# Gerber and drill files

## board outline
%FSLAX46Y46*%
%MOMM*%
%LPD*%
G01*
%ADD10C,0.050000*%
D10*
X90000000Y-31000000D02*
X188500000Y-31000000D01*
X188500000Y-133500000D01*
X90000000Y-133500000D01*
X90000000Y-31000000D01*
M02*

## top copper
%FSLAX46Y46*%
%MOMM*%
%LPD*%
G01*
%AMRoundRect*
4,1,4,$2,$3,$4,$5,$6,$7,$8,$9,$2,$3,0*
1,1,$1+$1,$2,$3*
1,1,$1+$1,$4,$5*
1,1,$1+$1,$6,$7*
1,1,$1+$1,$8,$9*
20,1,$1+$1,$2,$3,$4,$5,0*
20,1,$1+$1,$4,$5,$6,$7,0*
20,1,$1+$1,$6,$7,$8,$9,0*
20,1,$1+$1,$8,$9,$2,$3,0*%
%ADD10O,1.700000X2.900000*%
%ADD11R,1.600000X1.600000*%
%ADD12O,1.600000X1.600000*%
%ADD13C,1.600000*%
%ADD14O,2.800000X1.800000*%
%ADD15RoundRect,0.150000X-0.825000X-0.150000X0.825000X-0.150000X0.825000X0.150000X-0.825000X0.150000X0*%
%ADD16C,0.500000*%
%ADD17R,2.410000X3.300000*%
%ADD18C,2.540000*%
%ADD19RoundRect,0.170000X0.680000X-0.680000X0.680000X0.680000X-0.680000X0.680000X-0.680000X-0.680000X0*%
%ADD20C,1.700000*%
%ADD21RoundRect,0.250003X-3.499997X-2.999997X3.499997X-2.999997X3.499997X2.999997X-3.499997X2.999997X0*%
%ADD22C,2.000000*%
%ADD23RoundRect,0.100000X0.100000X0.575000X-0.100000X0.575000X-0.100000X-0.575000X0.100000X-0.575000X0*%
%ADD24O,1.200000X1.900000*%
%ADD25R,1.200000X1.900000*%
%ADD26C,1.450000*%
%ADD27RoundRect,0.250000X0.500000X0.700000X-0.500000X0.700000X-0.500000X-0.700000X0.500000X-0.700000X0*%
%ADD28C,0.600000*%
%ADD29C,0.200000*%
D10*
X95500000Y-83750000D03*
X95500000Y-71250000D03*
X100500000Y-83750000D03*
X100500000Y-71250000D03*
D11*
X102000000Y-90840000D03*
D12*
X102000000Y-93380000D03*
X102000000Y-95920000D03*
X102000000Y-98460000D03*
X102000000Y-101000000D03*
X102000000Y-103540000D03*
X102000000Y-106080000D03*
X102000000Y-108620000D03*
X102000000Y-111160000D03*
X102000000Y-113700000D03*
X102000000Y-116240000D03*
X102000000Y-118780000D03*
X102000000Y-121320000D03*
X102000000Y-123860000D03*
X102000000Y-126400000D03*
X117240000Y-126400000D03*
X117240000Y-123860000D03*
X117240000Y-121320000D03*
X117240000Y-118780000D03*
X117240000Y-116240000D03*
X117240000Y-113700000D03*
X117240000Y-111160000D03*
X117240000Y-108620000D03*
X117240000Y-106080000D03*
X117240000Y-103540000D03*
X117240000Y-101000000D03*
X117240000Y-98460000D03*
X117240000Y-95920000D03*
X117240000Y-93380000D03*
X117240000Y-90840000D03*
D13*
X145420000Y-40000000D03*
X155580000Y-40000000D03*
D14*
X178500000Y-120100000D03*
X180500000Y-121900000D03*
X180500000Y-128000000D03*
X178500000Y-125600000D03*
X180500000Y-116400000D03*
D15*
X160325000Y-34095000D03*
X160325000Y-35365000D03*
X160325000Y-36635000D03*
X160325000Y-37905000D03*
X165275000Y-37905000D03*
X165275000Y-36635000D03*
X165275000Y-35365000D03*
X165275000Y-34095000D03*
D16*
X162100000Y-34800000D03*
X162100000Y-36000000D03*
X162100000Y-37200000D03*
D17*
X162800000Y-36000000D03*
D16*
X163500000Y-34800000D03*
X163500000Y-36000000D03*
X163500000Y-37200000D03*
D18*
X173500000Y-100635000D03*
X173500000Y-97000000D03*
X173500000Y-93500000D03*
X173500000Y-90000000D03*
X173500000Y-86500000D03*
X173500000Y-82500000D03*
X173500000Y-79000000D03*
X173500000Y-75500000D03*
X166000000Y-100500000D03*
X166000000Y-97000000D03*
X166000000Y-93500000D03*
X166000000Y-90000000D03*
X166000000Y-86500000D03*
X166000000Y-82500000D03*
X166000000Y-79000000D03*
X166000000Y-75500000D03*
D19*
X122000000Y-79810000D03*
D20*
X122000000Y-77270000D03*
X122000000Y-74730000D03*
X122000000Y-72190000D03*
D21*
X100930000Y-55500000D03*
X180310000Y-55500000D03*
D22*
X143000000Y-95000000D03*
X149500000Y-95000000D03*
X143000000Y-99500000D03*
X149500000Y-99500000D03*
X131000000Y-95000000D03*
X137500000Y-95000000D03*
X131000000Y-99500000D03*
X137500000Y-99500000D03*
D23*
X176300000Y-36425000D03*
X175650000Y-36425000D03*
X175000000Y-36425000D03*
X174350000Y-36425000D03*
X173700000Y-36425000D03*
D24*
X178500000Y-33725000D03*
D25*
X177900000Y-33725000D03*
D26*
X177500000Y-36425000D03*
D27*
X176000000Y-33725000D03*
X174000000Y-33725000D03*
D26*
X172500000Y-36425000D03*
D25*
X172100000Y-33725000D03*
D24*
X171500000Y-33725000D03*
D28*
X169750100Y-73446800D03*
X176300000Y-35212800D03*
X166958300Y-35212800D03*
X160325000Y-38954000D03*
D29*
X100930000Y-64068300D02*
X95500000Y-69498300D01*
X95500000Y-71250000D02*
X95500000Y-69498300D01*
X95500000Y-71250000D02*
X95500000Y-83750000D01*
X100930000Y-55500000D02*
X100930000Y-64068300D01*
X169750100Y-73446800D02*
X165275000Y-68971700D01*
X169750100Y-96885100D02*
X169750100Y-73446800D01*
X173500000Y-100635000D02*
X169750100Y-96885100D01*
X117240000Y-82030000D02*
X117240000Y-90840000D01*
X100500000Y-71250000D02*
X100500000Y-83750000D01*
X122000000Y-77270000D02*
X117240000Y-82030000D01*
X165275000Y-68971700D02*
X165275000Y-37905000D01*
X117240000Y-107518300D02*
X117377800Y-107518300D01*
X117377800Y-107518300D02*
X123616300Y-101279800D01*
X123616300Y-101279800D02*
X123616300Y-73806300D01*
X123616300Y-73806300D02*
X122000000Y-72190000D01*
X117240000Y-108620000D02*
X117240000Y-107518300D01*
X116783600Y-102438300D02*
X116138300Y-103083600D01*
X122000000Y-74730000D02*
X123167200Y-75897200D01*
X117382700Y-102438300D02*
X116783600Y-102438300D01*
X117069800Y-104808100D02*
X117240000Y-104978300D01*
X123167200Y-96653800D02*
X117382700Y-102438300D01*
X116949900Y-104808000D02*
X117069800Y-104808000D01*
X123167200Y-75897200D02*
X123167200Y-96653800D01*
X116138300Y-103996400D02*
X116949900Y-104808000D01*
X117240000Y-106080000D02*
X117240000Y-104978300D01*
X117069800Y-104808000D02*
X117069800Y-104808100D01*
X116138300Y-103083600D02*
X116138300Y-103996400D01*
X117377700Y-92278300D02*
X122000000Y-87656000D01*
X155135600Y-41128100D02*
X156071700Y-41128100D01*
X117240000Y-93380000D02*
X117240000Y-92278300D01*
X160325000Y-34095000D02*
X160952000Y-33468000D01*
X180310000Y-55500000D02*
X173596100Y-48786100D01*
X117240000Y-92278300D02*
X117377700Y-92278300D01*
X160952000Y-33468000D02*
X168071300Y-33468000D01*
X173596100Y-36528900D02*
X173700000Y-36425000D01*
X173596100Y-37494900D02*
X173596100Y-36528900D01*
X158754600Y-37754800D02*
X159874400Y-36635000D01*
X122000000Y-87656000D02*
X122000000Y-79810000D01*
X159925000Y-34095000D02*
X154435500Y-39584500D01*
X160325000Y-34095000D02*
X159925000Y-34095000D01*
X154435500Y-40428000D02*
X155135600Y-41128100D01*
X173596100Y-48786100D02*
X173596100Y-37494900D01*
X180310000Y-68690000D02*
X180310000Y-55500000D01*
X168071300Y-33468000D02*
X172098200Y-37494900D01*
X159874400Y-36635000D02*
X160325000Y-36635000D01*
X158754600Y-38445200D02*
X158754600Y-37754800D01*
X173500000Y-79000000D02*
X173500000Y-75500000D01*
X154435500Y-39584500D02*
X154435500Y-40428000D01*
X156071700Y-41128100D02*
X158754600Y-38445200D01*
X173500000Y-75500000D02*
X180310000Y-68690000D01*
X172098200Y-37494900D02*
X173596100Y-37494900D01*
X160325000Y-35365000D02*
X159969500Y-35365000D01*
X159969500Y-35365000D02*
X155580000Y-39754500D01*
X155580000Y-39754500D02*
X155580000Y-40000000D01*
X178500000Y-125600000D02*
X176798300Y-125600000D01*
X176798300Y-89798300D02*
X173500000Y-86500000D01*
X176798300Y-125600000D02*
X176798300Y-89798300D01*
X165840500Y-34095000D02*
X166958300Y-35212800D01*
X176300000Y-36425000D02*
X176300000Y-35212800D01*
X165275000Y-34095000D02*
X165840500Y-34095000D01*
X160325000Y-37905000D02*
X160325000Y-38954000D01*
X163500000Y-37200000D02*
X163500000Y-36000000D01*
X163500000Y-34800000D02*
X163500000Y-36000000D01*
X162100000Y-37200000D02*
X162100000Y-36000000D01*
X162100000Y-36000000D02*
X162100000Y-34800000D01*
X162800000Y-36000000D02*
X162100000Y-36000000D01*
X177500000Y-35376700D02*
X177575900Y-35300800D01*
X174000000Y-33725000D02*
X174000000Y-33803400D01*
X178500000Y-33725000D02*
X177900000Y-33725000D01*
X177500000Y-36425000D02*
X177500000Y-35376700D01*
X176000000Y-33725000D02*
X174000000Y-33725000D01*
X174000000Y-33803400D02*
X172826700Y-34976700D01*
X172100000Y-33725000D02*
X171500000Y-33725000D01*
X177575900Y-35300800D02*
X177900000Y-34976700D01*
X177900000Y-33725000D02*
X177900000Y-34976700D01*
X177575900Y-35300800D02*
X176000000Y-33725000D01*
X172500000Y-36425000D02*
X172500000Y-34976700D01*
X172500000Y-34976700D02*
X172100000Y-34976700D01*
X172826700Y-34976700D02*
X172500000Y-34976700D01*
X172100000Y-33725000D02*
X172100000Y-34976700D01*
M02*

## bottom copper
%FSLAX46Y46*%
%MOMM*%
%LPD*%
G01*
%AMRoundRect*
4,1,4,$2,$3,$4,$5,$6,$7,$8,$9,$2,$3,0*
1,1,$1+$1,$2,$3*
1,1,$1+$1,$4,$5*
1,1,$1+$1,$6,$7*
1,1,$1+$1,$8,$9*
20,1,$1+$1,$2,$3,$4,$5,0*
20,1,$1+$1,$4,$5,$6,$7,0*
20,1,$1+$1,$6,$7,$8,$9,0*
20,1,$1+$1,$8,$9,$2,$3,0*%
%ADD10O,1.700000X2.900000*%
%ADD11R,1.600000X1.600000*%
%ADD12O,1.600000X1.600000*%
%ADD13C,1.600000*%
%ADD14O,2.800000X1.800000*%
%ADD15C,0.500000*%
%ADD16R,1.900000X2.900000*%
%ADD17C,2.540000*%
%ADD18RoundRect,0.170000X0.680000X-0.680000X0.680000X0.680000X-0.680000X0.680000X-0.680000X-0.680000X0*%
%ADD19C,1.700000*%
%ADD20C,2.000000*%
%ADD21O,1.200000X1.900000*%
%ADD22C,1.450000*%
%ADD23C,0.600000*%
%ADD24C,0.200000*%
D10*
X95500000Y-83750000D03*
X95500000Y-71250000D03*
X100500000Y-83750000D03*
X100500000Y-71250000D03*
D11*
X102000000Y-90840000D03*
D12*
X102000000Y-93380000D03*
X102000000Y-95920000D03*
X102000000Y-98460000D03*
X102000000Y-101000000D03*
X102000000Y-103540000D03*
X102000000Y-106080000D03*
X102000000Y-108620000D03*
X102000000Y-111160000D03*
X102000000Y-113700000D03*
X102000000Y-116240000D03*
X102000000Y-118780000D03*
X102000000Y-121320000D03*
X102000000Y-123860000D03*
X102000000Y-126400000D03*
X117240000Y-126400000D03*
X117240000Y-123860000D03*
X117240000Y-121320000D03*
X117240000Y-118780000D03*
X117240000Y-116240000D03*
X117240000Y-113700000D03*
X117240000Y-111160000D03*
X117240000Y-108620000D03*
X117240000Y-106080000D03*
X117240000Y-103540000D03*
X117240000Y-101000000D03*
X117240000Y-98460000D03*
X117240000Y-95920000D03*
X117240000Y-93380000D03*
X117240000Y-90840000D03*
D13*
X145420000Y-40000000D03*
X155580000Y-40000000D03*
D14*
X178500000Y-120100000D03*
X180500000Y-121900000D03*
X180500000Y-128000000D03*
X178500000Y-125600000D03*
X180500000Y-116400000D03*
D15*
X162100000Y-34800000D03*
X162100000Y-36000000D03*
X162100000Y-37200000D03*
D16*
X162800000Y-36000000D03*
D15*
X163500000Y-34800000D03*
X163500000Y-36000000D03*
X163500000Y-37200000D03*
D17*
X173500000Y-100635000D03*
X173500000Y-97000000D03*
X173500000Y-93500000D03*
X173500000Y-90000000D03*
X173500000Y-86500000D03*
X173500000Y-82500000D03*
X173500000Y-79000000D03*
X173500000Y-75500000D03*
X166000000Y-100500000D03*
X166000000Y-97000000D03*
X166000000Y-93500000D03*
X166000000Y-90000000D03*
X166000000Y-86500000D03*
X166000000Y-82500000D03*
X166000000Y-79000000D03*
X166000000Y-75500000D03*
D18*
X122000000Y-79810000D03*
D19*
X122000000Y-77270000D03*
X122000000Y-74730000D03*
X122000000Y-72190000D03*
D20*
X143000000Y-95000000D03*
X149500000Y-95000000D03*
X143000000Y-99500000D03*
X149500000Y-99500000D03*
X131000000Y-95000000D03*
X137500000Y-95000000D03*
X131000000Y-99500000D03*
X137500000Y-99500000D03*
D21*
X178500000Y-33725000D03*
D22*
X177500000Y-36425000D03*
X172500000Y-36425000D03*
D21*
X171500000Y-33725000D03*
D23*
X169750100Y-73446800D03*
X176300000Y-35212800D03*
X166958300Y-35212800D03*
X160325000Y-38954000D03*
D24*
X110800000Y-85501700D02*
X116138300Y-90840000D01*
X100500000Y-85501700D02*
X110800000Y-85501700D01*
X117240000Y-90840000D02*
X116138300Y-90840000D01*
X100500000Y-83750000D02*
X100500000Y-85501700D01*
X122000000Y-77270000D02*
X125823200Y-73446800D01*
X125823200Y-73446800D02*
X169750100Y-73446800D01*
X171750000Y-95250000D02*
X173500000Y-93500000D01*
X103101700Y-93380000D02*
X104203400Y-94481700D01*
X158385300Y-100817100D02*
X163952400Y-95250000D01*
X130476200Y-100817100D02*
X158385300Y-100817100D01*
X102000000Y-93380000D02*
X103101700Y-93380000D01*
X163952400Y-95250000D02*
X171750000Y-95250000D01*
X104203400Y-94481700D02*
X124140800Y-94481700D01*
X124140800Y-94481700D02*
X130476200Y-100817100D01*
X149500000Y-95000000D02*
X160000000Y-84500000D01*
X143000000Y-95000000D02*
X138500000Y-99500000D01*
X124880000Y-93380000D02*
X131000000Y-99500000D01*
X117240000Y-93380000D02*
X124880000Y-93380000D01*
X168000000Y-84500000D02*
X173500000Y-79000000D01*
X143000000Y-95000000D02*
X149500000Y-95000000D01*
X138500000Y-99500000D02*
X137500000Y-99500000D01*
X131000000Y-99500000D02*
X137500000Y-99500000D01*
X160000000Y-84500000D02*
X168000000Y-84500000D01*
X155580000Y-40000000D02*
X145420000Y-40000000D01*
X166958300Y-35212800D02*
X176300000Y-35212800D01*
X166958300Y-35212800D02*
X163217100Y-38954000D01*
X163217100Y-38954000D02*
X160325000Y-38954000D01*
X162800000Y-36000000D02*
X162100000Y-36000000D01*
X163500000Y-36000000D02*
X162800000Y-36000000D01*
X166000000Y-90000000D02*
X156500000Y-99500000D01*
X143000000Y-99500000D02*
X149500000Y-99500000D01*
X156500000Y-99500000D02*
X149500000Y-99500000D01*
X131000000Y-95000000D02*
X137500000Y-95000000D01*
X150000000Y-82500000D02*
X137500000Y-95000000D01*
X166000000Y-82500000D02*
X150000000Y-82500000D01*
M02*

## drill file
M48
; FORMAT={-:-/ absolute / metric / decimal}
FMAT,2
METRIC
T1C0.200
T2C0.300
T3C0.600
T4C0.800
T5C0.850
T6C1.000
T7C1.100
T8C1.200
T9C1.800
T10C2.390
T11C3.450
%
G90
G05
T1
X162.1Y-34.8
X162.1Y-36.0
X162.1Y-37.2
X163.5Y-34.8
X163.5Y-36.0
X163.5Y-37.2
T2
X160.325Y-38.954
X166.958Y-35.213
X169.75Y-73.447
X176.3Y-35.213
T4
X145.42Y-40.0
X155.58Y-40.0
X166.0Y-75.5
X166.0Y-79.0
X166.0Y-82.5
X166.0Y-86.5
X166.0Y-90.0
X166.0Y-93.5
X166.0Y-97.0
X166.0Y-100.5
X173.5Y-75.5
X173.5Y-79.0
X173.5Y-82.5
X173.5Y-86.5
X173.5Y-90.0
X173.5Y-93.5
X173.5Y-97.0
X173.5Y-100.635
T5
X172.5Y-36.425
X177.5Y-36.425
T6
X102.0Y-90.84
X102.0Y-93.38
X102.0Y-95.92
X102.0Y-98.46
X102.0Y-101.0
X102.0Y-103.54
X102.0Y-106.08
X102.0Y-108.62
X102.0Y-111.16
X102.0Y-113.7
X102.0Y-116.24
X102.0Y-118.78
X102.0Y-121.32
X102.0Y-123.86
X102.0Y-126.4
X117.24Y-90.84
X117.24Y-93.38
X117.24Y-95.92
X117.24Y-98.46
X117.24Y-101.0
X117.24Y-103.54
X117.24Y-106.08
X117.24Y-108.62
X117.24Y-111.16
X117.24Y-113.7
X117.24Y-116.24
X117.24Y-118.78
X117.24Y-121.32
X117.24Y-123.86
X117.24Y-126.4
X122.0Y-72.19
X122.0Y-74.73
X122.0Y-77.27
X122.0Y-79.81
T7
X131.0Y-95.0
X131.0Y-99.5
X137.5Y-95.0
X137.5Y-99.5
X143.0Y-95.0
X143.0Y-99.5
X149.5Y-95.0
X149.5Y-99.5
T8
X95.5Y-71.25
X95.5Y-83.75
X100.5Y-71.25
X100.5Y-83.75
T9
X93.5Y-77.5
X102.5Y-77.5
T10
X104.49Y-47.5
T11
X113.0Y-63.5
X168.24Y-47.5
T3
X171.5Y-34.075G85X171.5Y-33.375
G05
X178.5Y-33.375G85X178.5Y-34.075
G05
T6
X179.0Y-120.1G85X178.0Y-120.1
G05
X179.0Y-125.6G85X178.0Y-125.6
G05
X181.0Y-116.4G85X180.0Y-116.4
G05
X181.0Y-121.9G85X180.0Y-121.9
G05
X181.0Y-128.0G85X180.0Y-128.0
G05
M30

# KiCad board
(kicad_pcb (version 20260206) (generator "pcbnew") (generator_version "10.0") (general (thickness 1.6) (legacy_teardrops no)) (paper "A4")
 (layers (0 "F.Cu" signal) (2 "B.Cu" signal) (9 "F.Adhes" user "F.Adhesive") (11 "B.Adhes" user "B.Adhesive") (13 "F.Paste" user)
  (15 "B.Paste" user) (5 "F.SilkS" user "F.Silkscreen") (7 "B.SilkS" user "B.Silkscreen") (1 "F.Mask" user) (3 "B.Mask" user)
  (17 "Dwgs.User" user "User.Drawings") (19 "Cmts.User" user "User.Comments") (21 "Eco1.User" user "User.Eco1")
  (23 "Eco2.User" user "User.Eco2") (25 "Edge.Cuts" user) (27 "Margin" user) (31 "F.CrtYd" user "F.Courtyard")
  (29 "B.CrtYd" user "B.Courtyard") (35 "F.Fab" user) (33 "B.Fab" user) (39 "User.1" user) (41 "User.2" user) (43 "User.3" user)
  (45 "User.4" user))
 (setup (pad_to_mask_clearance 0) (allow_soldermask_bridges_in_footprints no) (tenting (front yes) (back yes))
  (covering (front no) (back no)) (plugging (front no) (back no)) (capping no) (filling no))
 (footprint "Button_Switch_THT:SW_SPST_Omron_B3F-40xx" (layer "F.Cu") (at 95.5 83.75 90)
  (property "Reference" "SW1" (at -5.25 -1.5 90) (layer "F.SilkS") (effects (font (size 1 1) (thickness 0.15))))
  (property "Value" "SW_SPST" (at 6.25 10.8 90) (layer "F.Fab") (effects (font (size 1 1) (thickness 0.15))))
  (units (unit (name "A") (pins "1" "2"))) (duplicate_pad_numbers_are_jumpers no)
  (pad "" np_thru_hole circle (at 6.25 -2 90) (size 1.8 1.8) (drill 1.8) (layers "*.Cu" "*.Mask"))
  (pad "" np_thru_hole circle (at 6.25 7 90) (size 1.8 1.8) (drill 1.8) (layers "*.Cu" "*.Mask"))
  (pad "1" thru_hole oval (at 0 0 90) (size 2.9 1.7) (drill 1.2) (layers "*.Cu" "*.Mask") (remove_unused_layers no) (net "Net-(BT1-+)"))
  (pad "1" thru_hole oval (at 12.5 0 90) (size 2.9 1.7) (drill 1.2) (layers "*.Cu" "*.Mask") (remove_unused_layers no) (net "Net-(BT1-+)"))
  (pad "2" thru_hole oval (at 0 5 90) (size 2.9 1.7) (drill 1.2) (layers "*.Cu" "*.Mask") (remove_unused_layers no) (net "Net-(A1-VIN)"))
  (pad "2" thru_hole oval (at 12.5 5 90) (size 2.9 1.7) (drill 1.2) (layers "*.Cu" "*.Mask") (remove_unused_layers no) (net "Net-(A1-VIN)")))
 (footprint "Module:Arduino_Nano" (layer "F.Cu") (at 102 90.84)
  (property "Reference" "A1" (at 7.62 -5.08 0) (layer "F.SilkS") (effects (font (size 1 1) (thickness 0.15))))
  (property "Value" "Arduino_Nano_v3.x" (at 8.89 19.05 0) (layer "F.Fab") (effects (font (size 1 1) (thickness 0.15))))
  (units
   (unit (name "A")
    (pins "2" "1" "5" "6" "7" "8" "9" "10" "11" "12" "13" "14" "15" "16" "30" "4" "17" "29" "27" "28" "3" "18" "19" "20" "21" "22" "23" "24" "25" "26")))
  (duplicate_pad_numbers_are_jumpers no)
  (pad "1" thru_hole rect (at 0 0) (size 1.6 1.6) (drill 1) (layers "*.Cu" "*.Mask") (remove_unused_layers no)
   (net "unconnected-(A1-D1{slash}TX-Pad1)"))
  (pad "2" thru_hole oval (at 0 2.54) (size 1.6 1.6) (drill 1) (layers "*.Cu" "*.Mask") (remove_unused_layers no)
   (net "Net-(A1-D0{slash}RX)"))
  (pad "3" thru_hole oval (at 0 5.08) (size 1.6 1.6) (drill 1) (layers "*.Cu" "*.Mask") (remove_unused_layers no)
   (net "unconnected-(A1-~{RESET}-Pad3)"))
  (pad "4" thru_hole oval (at 0 7.62) (size 1.6 1.6) (drill 1) (layers "*.Cu" "*.Mask") (remove_unused_layers no)
   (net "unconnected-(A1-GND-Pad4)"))
  (pad "5" thru_hole oval (at 0 10.16) (size 1.6 1.6) (drill 1) (layers "*.Cu" "*.Mask") (remove_unused_layers no)
   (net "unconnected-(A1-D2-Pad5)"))
  (pad "6" thru_hole oval (at 0 12.7) (size 1.6 1.6) (drill 1) (layers "*.Cu" "*.Mask") (remove_unused_layers no)
   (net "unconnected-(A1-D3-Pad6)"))
  (pad "7" thru_hole oval (at 0 15.24) (size 1.6 1.6) (drill 1) (layers "*.Cu" "*.Mask") (remove_unused_layers no)
   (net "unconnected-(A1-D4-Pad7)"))
  (pad "8" thru_hole oval (at 0 17.78) (size 1.6 1.6) (drill 1) (layers "*.Cu" "*.Mask") (remove_unused_layers no)
   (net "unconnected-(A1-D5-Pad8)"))
  (pad "9" thru_hole oval (at 0 20.32) (size 1.6 1.6) (drill 1) (layers "*.Cu" "*.Mask") (remove_unused_layers no)
   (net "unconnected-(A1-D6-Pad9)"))
  (pad "10" thru_hole oval (at 0 22.86) (size 1.6 1.6) (drill 1) (layers "*.Cu" "*.Mask") (remove_unused_layers no)
   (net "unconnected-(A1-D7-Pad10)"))
  (pad "11" thru_hole oval (at 0 25.4) (size 1.6 1.6) (drill 1) (layers "*.Cu" "*.Mask") (remove_unused_layers no)
   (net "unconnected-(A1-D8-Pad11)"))
  (pad "12" thru_hole oval (at 0 27.94) (size 1.6 1.6) (drill 1) (layers "*.Cu" "*.Mask") (remove_unused_layers no)
   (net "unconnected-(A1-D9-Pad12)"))
  (pad "13" thru_hole oval (at 0 30.48) (size 1.6 1.6) (drill 1) (layers "*.Cu" "*.Mask") (remove_unused_layers no)
   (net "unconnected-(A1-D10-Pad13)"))
  (pad "14" thru_hole oval (at 0 33.02) (size 1.6 1.6) (drill 1) (layers "*.Cu" "*.Mask") (remove_unused_layers no)
   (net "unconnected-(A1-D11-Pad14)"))
  (pad "15" thru_hole oval (at 0 35.56) (size 1.6 1.6) (drill 1) (layers "*.Cu" "*.Mask") (remove_unused_layers no)
   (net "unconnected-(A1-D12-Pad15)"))
  (pad "16" thru_hole oval (at 15.24 35.56) (size 1.6 1.6) (drill 1) (layers "*.Cu" "*.Mask") (remove_unused_layers no)
   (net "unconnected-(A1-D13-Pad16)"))
  (pad "17" thru_hole oval (at 15.24 33.02) (size 1.6 1.6) (drill 1) (layers "*.Cu" "*.Mask") (remove_unused_layers no)
   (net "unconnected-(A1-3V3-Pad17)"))
  (pad "18" thru_hole oval (at 15.24 30.48) (size 1.6 1.6) (drill 1) (layers "*.Cu" "*.Mask") (remove_unused_layers no)
   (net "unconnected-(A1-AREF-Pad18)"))
  (pad "19" thru_hole oval (at 15.24 27.94) (size 1.6 1.6) (drill 1) (layers "*.Cu" "*.Mask") (remove_unused_layers no)
   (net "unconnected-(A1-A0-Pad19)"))
  (pad "20" thru_hole oval (at 15.24 25.4) (size 1.6 1.6) (drill 1) (layers "*.Cu" "*.Mask") (remove_unused_layers no)
   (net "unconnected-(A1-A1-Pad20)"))
  (pad "21" thru_hole oval (at 15.24 22.86) (size 1.6 1.6) (drill 1) (layers "*.Cu" "*.Mask") (remove_unused_layers no)
   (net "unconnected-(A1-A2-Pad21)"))
  (pad "22" thru_hole oval (at 15.24 20.32) (size 1.6 1.6) (drill 1) (layers "*.Cu" "*.Mask") (remove_unused_layers no)
   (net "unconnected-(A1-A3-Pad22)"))
  (pad "23" thru_hole oval (at 15.24 17.78) (size 1.6 1.6) (drill 1) (layers "*.Cu" "*.Mask") (remove_unused_layers no) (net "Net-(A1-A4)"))
  (pad "24" thru_hole oval (at 15.24 15.24) (size 1.6 1.6) (drill 1) (layers "*.Cu" "*.Mask") (remove_unused_layers no) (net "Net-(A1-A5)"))
  (pad "25" thru_hole oval (at 15.24 12.7) (size 1.6 1.6) (drill 1) (layers "*.Cu" "*.Mask") (remove_unused_layers no)
   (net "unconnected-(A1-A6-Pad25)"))
  (pad "26" thru_hole oval (at 15.24 10.16) (size 1.6 1.6) (drill 1) (layers "*.Cu" "*.Mask") (remove_unused_layers no)
   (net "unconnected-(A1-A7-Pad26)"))
  (pad "27" thru_hole oval (at 15.24 7.62) (size 1.6 1.6) (drill 1) (layers "*.Cu" "*.Mask") (remove_unused_layers no)
   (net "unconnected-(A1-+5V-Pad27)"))
  (pad "28" thru_hole oval (at 15.24 5.08) (size 1.6 1.6) (drill 1) (layers "*.Cu" "*.Mask") (remove_unused_layers no)
   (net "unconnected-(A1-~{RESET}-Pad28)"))
  (pad "29" thru_hole oval (at 15.24 2.54) (size 1.6 1.6) (drill 1) (layers "*.Cu" "*.Mask") (remove_unused_layers no) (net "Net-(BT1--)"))
  (pad "30" thru_hole oval (at 15.24 0) (size 1.6 1.6) (drill 1) (layers "*.Cu" "*.Mask") (remove_unused_layers no) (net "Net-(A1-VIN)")))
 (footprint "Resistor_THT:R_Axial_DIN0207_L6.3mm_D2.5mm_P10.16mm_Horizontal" (layer "F.Cu") (at 145.42 40)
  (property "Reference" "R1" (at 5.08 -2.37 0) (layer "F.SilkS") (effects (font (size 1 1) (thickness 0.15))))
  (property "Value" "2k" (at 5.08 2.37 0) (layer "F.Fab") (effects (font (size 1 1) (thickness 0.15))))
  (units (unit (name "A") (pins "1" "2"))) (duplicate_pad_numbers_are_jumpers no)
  (pad "1" thru_hole circle (at 0 0) (size 1.6 1.6) (drill 0.8) (layers "*.Cu" "*.Mask") (remove_unused_layers no) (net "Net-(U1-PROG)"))
  (pad "2" thru_hole circle (at 10.16 0) (size 1.6 1.6) (drill 0.8) (layers "*.Cu" "*.Mask") (remove_unused_layers no) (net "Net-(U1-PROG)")))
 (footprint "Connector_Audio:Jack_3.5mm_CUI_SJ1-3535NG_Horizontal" (layer "F.Cu") (at 180.5 128 180)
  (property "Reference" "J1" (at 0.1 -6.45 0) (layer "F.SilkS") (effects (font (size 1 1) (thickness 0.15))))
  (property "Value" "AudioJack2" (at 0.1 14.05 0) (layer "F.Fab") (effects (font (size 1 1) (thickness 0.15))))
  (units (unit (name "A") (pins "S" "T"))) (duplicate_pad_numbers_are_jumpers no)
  (pad "R" thru_hole oval (at 2 7.9 180) (size 2.8 1.8) (drill oval 2 1) (layers "*.Cu" "*.Mask") (remove_unused_layers no))
  (pad "RN" thru_hole oval (at 0 6.1 180) (size 2.8 1.8) (drill oval 2 1) (layers "*.Cu" "*.Mask") (remove_unused_layers no))
  (pad "S" thru_hole oval (at 0 0 180) (size 2.8 1.8) (drill oval 2 1) (layers "*.Cu" "*.Mask") (remove_unused_layers no)
   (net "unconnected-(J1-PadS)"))
  (pad "T" thru_hole oval (at 2 2.4 180) (size 2.8 1.8) (drill oval 2 1) (layers "*.Cu" "*.Mask") (remove_unused_layers no)
   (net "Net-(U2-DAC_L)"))
  (pad "TN" thru_hole oval (at 0 11.6 180) (size 2.8 1.8) (drill oval 2 1) (layers "*.Cu" "*.Mask") (remove_unused_layers no)))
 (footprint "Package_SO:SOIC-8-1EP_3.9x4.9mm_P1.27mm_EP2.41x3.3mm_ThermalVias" (layer "F.Cu") (at 162.8 36)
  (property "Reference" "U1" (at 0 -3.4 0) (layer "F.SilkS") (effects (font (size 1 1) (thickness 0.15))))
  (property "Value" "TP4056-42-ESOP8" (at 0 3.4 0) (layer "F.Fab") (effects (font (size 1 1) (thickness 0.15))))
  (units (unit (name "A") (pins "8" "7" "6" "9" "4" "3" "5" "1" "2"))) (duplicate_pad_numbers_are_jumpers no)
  (pad "" smd roundrect (at -0.6 -0.825) (size 1.01 1.38) (layers "F.Paste") (roundrect_rratio 0.247525))
  (pad "" smd roundrect (at -0.6 0.825) (size 1.01 1.38) (layers "F.Paste") (roundrect_rratio 0.247525))
  (pad "" smd roundrect (at 0.6 -0.825) (size 1.01 1.38) (layers "F.Paste") (roundrect_rratio 0.247525))
  (pad "" smd roundrect (at 0.6 0.825) (size 1.01 1.38) (layers "F.Paste") (roundrect_rratio 0.247525))
  (pad "1" smd roundrect (at -2.475 -1.905) (size 1.95 0.6) (layers "F.Cu" "F.Mask" "F.Paste") (roundrect_rratio 0.25) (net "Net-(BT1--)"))
  (pad "2" smd roundrect (at -2.475 -0.635) (size 1.95 0.6) (layers "F.Cu" "F.Mask" "F.Paste") (roundrect_rratio 0.25) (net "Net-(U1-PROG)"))
  (pad "3" smd roundrect (at -2.475 0.635) (size 1.95 0.6) (layers "F.Cu" "F.Mask" "F.Paste") (roundrect_rratio 0.25) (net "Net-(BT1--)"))
  (pad "4" smd roundrect (at -2.475 1.905) (size 1.95 0.6) (layers "F.Cu" "F.Mask" "F.Paste") (roundrect_rratio 0.25) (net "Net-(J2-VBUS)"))
  (pad "5" smd roundrect (at 2.475 1.905) (size 1.95 0.6) (layers "F.Cu" "F.Mask" "F.Paste") (roundrect_rratio 0.25) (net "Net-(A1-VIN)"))
  (pad "6" smd roundrect (at 2.475 0.635) (size 1.95 0.6) (layers "F.Cu" "F.Mask" "F.Paste") (roundrect_rratio 0.25)
   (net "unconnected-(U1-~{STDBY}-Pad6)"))
  (pad "7" smd roundrect (at 2.475 -0.635) (size 1.95 0.6) (layers "F.Cu" "F.Mask" "F.Paste") (roundrect_rratio 0.25)
   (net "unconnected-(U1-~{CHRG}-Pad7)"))
  (pad "8" smd roundrect (at 2.475 -1.905) (size 1.95 0.6) (layers "F.Cu" "F.Mask" "F.Paste") (roundrect_rratio 0.25) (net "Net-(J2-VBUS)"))
  (pad "9" thru_hole circle (at -0.7 -1.2) (size 0.5 0.5) (drill 0.2) (layers "*.Cu") (remove_unused_layers no)
   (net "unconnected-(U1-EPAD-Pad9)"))
  (pad "9" thru_hole circle (at -0.7 0) (size 0.5 0.5) (drill 0.2) (layers "*.Cu") (remove_unused_layers no)
   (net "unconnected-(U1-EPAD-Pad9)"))
  (pad "9" thru_hole circle (at -0.7 1.2) (size 0.5 0.5) (drill 0.2) (layers "*.Cu") (remove_unused_layers no)
   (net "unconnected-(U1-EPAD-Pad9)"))
  (pad "9" smd rect (at 0 0) (size 1.9 2.9) (layers "B.Cu") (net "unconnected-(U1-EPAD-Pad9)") (zone_connect 2))
  (pad "9" smd rect (at 0 0) (size 2.41 3.3) (layers "F.Cu" "F.Mask") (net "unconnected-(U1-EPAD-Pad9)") (zone_connect 2))
  (pad "9" thru_hole circle (at 0.7 -1.2) (size 0.5 0.5) (drill 0.2) (layers "*.Cu") (remove_unused_layers no)
   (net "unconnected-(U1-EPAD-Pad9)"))
  (pad "9" thru_hole circle (at 0.7 0) (size 0.5 0.5) (drill 0.2) (layers "*.Cu") (remove_unused_layers no)
   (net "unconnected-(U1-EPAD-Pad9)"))
  (pad "9" thru_hole circle (at 0.7 1.2) (size 0.5 0.5) (drill 0.2) (layers "*.Cu") (remove_unused_layers no)
   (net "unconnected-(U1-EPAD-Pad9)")))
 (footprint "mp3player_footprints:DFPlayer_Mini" (layer "F.Cu") (at 183.5 91.5 180)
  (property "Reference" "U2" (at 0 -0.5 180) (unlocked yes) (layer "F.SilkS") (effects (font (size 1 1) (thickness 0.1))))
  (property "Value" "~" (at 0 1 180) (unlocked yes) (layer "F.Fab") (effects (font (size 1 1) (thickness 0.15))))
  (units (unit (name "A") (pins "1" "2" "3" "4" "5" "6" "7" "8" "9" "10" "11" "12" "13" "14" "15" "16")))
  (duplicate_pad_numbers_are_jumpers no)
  (pad "1" thru_hole circle (at 10 -9.135 180) (size 2.54 2.54) (drill 0.8) (layers "*.Cu" "*.Mask") (remove_unused_layers no)
   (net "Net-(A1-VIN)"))
  (pad "2" thru_hole circle (at 10 -5.5 180) (size 2.54 2.54) (drill 0.8) (layers "*.Cu" "*.Mask") (remove_unused_layers no)
   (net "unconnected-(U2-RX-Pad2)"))
  (pad "3" thru_hole circle (at 10 -2 180) (size 2.54 2.54) (drill 0.8) (layers "*.Cu" "*.Mask") (remove_unused_layers no)
   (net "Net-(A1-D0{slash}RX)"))
  (pad "4" thru_hole circle (at 10 1.5 180) (size 2.54 2.54) (drill 0.8) (layers "*.Cu" "*.Mask") (remove_unused_layers no)
   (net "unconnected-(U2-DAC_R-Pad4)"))
  (pad "5" thru_hole circle (at 10 5 180) (size 2.54 2.54) (drill 0.8) (layers "*.Cu" "*.Mask") (remove_unused_layers no)
   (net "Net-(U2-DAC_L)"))
  (pad "6" thru_hole circle (at 10 9 180) (size 2.54 2.54) (drill 0.8) (layers "*.Cu" "*.Mask") (remove_unused_layers no)
   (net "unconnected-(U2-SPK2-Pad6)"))
  (pad "7" thru_hole circle (at 10 12.5 180) (size 2.54 2.54) (drill 0.8) (layers "*.Cu" "*.Mask") (remove_unused_layers no)
   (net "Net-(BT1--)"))
  (pad "8" thru_hole circle (at 10 16 180) (size 2.54 2.54) (drill 0.8) (layers "*.Cu" "*.Mask") (remove_unused_layers no)
   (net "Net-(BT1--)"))
  (pad "9" thru_hole circle (at 17.5 -9 180) (size 2.54 2.54) (drill 0.8) (layers "*.Cu" "*.Mask") (remove_unused_layers no)
   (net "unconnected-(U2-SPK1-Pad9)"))
  (pad "10" thru_hole circle (at 17.5 -5.5 180) (size 2.54 2.54) (drill 0.8) (layers "*.Cu" "*.Mask") (remove_unused_layers no)
   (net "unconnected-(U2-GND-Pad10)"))
  (pad "11" thru_hole circle (at 17.5 -2 180) (size 2.54 2.54) (drill 0.8) (layers "*.Cu" "*.Mask") (remove_unused_layers no)
   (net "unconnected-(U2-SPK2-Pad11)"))
  (pad "12" thru_hole circle (at 17.5 1.5 180) (size 2.54 2.54) (drill 0.8) (layers "*.Cu" "*.Mask") (remove_unused_layers no)
   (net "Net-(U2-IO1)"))
  (pad "13" thru_hole circle (at 17.5 5 180) (size 2.54 2.54) (drill 0.8) (layers "*.Cu" "*.Mask") (remove_unused_layers no)
   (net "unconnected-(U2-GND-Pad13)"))
  (pad "14" thru_hole circle (at 17.5 9 180) (size 2.54 2.54) (drill 0.8) (layers "*.Cu" "*.Mask") (remove_unused_layers no)
   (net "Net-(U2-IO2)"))
  (pad "15" thru_hole circle (at 17.5 12.5 180) (size 2.54 2.54) (drill 0.8) (layers "*.Cu" "*.Mask") (remove_unused_layers no)
   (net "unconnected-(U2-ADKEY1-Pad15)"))
  (pad "16" thru_hole circle (at 17.5 16 180) (size 2.54 2.54) (drill 0.8) (layers "*.Cu" "*.Mask") (remove_unused_layers no)
   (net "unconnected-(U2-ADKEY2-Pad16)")))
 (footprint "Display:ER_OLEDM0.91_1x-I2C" (layer "F.Cu") (at 122 79.81 90)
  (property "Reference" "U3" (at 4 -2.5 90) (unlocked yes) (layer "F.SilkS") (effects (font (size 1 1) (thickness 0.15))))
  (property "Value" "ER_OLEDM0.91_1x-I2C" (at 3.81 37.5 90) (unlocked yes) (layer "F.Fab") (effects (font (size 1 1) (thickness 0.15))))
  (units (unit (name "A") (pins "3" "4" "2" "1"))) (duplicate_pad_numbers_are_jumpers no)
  (pad "1" thru_hole roundrect (at 0 0 90) (size 1.7 1.7) (drill 1) (layers "*.Cu" "*.Mask") (remove_unused_layers no)
   (roundrect_rratio 0.1) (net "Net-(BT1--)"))
  (pad "2" thru_hole circle (at 2.54 0 90) (size 1.7 1.7) (drill 1) (layers "*.Cu" "*.Mask") (remove_unused_layers no) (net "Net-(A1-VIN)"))
  (pad "3" thru_hole circle (at 5.08 0 90) (size 1.7 1.7) (drill 1) (layers "*.Cu" "*.Mask") (remove_unused_layers no) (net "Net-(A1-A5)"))
  (pad "4" thru_hole circle (at 7.62 0 90) (size 1.7 1.7) (drill 1) (layers "*.Cu" "*.Mask") (remove_unused_layers no) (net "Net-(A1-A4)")))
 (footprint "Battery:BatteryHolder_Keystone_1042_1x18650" (layer "F.Cu") (at 140.62 55.5)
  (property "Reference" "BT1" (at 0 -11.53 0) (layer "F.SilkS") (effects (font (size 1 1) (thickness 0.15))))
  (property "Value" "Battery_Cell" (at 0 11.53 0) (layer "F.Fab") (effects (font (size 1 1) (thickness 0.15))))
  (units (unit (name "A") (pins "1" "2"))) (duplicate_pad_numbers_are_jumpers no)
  (pad "" np_thru_hole circle (at -36.13 -8) (size 2.39 2.39) (drill 2.39) (layers "*.Cu" "*.Mask"))
  (pad "" np_thru_hole circle (at -27.62 8) (size 3.45 3.45) (drill 3.45) (layers "*.Cu" "*.Mask"))
  (pad "" np_thru_hole circle (at 27.62 -8) (size 3.45 3.45) (drill 3.45) (layers "*.Cu" "*.Mask"))
  (pad "1" smd roundrect (at -39.69 0) (size 7.5 6.5) (layers "F.Cu" "F.Mask" "F.Paste") (roundrect_rratio 0.038462) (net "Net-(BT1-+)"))
  (pad "2" smd roundrect (at 39.69 0) (size 7.5 6.5) (layers "F.Cu" "F.Mask" "F.Paste") (roundrect_rratio 0.038462) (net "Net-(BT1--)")))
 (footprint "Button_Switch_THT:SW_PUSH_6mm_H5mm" (layer "F.Cu") (at 143 95)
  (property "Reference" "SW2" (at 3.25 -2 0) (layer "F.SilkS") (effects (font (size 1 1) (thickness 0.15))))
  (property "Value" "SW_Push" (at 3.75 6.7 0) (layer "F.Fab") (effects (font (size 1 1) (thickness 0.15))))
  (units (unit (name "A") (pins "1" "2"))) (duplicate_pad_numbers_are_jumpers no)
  (pad "1" thru_hole circle (at 0 0 90) (size 2 2) (drill 1.1) (layers "*.Cu" "*.Mask") (remove_unused_layers no) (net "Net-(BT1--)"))
  (pad "1" thru_hole circle (at 6.5 0 90) (size 2 2) (drill 1.1) (layers "*.Cu" "*.Mask") (remove_unused_layers no) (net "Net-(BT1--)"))
  (pad "2" thru_hole circle (at 0 4.5 90) (size 2 2) (drill 1.1) (layers "*.Cu" "*.Mask") (remove_unused_layers no) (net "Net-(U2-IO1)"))
  (pad "2" thru_hole circle (at 6.5 4.5 90) (size 2 2) (drill 1.1) (layers "*.Cu" "*.Mask") (remove_unused_layers no) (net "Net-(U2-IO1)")))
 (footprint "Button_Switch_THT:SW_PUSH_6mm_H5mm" (layer "F.Cu") (at 131 95)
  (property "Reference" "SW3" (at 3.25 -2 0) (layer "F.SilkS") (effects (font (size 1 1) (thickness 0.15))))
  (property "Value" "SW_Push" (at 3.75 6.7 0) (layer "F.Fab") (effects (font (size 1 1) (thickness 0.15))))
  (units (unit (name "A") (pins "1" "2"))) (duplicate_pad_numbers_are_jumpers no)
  (pad "1" thru_hole circle (at 0 0 90) (size 2 2) (drill 1.1) (layers "*.Cu" "*.Mask") (remove_unused_layers no) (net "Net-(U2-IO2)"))
  (pad "1" thru_hole circle (at 6.5 0 90) (size 2 2) (drill 1.1) (layers "*.Cu" "*.Mask") (remove_unused_layers no) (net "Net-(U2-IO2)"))
  (pad "2" thru_hole circle (at 0 4.5 90) (size 2 2) (drill 1.1) (layers "*.Cu" "*.Mask") (remove_unused_layers no) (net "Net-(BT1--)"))
  (pad "2" thru_hole circle (at 6.5 4.5 90) (size 2 2) (drill 1.1) (layers "*.Cu" "*.Mask") (remove_unused_layers no) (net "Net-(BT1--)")))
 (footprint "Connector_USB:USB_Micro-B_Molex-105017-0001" (layer "F.Cu") (at 175 34.9625 180)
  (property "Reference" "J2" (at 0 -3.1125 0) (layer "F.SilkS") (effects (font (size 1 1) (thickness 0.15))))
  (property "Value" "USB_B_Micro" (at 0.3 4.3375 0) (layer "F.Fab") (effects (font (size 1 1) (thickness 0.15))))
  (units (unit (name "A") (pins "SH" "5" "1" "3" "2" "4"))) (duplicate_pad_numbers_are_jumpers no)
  (pad "1" smd roundrect (at -1.3 -1.4625 180) (size 0.4 1.35) (layers "F.Cu" "F.Mask" "F.Paste") (roundrect_rratio 0.25)
   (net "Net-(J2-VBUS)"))
  (pad "2" smd roundrect (at -0.65 -1.4625 180) (size 0.4 1.35) (layers "F.Cu" "F.Mask" "F.Paste") (roundrect_rratio 0.25)
   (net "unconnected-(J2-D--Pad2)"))
  (pad "3" smd roundrect (at 0 -1.4625 180) (size 0.4 1.35) (layers "F.Cu" "F.Mask" "F.Paste") (roundrect_rratio 0.25)
   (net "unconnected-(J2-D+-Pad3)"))
  (pad "4" smd roundrect (at 0.65 -1.4625 180) (size 0.4 1.35) (layers "F.Cu" "F.Mask" "F.Paste") (roundrect_rratio 0.25)
   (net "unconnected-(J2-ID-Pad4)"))
  (pad "5" smd roundrect (at 1.3 -1.4625 180) (size 0.4 1.35) (layers "F.Cu" "F.Mask" "F.Paste") (roundrect_rratio 0.25) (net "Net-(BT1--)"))
  (pad "SH" thru_hole oval (at -3.5 1.2375) (size 1.2 1.9) (drill oval 0.6 1.3) (layers "*.Cu" "*.Mask") (remove_unused_layers no)
   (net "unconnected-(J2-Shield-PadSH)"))
  (pad "SH" smd rect (at -2.9 1.2375 180) (size 1.2 1.9) (layers "F.Cu" "F.Mask") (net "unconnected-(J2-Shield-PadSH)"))
  (pad "SH" thru_hole circle (at -2.5 -1.4625 180) (size 1.45 1.45) (drill 0.85) (layers "*.Cu" "*.Mask") (remove_unused_layers no)
   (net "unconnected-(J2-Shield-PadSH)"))
  (pad "SH" smd roundrect (at -1 1.2375 180) (size 1.5 1.9) (layers "F.Cu" "F.Mask" "F.Paste") (roundrect_rratio 0.1666666667)
   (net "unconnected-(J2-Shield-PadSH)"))
  (pad "SH" smd roundrect (at 1 1.2375 180) (size 1.5 1.9) (layers "F.Cu" "F.Mask" "F.Paste") (roundrect_rratio 0.1666666667)
   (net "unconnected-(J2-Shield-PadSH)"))
  (pad "SH" thru_hole circle (at 2.5 -1.4625 180) (size 1.45 1.45) (drill 0.85) (layers "*.Cu" "*.Mask") (remove_unused_layers no)
   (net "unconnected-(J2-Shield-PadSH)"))
  (pad "SH" smd rect (at 2.9 1.2375 180) (size 1.2 1.9) (layers "F.Cu" "F.Mask") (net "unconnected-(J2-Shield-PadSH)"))
  (pad "SH" thru_hole oval (at 3.5 1.2375 180) (size 1.2 1.9) (drill oval 0.6 1.3) (layers "*.Cu" "*.Mask") (remove_unused_layers no)
   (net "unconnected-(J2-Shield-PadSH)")))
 (gr_rect (start 90 31) (end 188.5 133.5) (stroke (width 0.05) (type default)) (fill no) (layer "Edge.Cuts"))
 (segment (start 100.93 64.0683) (end 95.5 69.4983) (width 0.2) (layer "F.Cu") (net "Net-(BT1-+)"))
 (segment (start 95.5 71.25) (end 95.5 69.4983) (width 0.2) (layer "F.Cu") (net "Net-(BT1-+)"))
 (segment (start 95.5 71.25) (end 95.5 83.75) (width 0.2) (layer "F.Cu") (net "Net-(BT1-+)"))
 (segment (start 100.93 55.5) (end 100.93 64.0683) (width 0.2) (layer "F.Cu") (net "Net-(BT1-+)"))
 (segment (start 169.7501 73.4468) (end 165.275 68.9717) (width 0.2) (layer "F.Cu") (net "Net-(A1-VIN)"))
 (segment (start 169.7501 96.8851) (end 169.7501 73.4468) (width 0.2) (layer "F.Cu") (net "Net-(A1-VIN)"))
 (segment (start 173.5 100.635) (end 169.7501 96.8851) (width 0.2) (layer "F.Cu") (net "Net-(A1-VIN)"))
 (segment (start 117.24 82.03) (end 117.24 90.84) (width 0.2) (layer "F.Cu") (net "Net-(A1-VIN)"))
 (segment (start 100.5 71.25) (end 100.5 83.75) (width 0.2) (layer "F.Cu") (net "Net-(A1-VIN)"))
 (segment (start 122 77.27) (end 117.24 82.03) (width 0.2) (layer "F.Cu") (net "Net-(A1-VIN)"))
 (segment (start 165.275 68.9717) (end 165.275 37.905) (width 0.2) (layer "F.Cu") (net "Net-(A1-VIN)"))
 (via (at 169.7501 73.4468) (size 0.6) (drill 0.3) (layers "F.Cu" "B.Cu") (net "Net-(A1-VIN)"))
 (segment (start 110.8 85.5017) (end 116.1383 90.84) (width 0.2) (layer "B.Cu") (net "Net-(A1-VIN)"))
 (segment (start 100.5 85.5017) (end 110.8 85.5017) (width 0.2) (layer "B.Cu") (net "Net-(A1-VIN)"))
 (segment (start 117.24 90.84) (end 116.1383 90.84) (width 0.2) (layer "B.Cu") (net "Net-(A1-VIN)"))
 (segment (start 100.5 83.75) (end 100.5 85.5017) (width 0.2) (layer "B.Cu") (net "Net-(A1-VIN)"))
 (segment (start 122 77.27) (end 125.8232 73.4468) (width 0.2) (layer "B.Cu") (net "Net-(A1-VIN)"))
 (segment (start 125.8232 73.4468) (end 169.7501 73.4468) (width 0.2) (layer "B.Cu") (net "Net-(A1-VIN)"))
 (segment (start 171.75 95.25) (end 173.5 93.5) (width 0.2) (layer "B.Cu") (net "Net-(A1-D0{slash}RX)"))
 (segment (start 103.1017 93.38) (end 104.2034 94.4817) (width 0.2) (layer "B.Cu") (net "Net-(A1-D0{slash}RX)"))
 (segment (start 158.3853 100.8171) (end 163.9524 95.25) (width 0.2) (layer "B.Cu") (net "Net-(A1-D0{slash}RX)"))
 (segment (start 130.4762 100.8171) (end 158.3853 100.8171) (width 0.2) (layer "B.Cu") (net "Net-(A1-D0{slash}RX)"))
 (segment (start 102 93.38) (end 103.1017 93.38) (width 0.2) (layer "B.Cu") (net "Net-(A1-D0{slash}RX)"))
 (segment (start 163.9524 95.25) (end 171.75 95.25) (width 0.2) (layer "B.Cu") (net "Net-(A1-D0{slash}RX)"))
 (segment (start 104.2034 94.4817) (end 124.1408 94.4817) (width 0.2) (layer "B.Cu") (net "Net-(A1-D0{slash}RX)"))
 (segment (start 124.1408 94.4817) (end 130.4762 100.8171) (width 0.2) (layer "B.Cu") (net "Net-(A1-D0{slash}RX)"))
 (segment (start 117.24 107.5183) (end 117.3778 107.5183) (width 0.2) (layer "F.Cu") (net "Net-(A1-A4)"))
 (segment (start 117.3778 107.5183) (end 123.6163 101.2798) (width 0.2) (layer "F.Cu") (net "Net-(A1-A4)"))
 (segment (start 123.6163 101.2798) (end 123.6163 73.8063) (width 0.2) (layer "F.Cu") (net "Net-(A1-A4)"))
 (segment (start 123.6163 73.8063) (end 122 72.19) (width 0.2) (layer "F.Cu") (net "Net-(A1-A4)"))
 (segment (start 117.24 108.62) (end 117.24 107.5183) (width 0.2) (layer "F.Cu") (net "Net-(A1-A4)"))
 (segment (start 116.7836 102.4383) (end 116.1383 103.0836) (width 0.2) (layer "F.Cu") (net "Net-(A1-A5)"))
 (segment (start 122 74.73) (end 123.1672 75.8972) (width 0.2) (layer "F.Cu") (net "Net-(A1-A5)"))
 (segment (start 117.3827 102.4383) (end 116.7836 102.4383) (width 0.2) (layer "F.Cu") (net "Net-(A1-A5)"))
 (segment (start 117.0698 104.8081) (end 117.24 104.9783) (width 0.2) (layer "F.Cu") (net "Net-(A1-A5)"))
 (segment (start 123.1672 96.6538) (end 117.3827 102.4383) (width 0.2) (layer "F.Cu") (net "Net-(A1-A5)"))
 (segment (start 116.9499 104.808) (end 117.0698 104.808) (width 0.2) (layer "F.Cu") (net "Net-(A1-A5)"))
 (segment (start 123.1672 75.8972) (end 123.1672 96.6538) (width 0.2) (layer "F.Cu") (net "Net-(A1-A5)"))
 (segment (start 116.1383 103.9964) (end 116.9499 104.808) (width 0.2) (layer "F.Cu") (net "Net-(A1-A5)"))
 (segment (start 117.24 106.08) (end 117.24 104.9783) (width 0.2) (layer "F.Cu") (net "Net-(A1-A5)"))
 (segment (start 117.0698 104.808) (end 117.0698 104.8081) (width 0.2) (layer "F.Cu") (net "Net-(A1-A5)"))
 (segment (start 116.1383 103.0836) (end 116.1383 103.9964) (width 0.2) (layer "F.Cu") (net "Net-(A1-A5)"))
 (segment (start 117.3777 92.2783) (end 122 87.656) (width 0.2) (layer "F.Cu") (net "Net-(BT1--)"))
 (segment (start 155.1356 41.1281) (end 156.0717 41.1281) (width 0.2) (layer "F.Cu") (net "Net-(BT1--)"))
 (segment (start 117.24 93.38) (end 117.24 92.2783) (width 0.2) (layer "F.Cu") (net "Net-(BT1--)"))
 (segment (start 160.325 34.095) (end 160.952 33.468) (width 0.2) (layer "F.Cu") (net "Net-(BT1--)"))
 (segment (start 180.31 55.5) (end 173.5961 48.7861) (width 0.2) (layer "F.Cu") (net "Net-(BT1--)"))
 (segment (start 117.24 92.2783) (end 117.3777 92.2783) (width 0.2) (layer "F.Cu") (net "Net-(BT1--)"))
 (segment (start 160.952 33.468) (end 168.0713 33.468) (width 0.2) (layer "F.Cu") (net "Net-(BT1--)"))
 (segment (start 173.5961 36.5289) (end 173.7 36.425) (width 0.2) (layer "F.Cu") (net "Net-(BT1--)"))
 (segment (start 173.5961 37.4949) (end 173.5961 36.5289) (width 0.2) (layer "F.Cu") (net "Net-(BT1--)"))
 (segment (start 158.7546 37.7548) (end 159.8744 36.635) (width 0.2) (layer "F.Cu") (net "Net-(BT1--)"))
 (segment (start 122 87.656) (end 122 79.81) (width 0.2) (layer "F.Cu") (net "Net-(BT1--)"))
 (segment (start 159.925 34.095) (end 154.4355 39.5845) (width 0.2) (layer "F.Cu") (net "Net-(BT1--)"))
 (segment (start 160.325 34.095) (end 159.925 34.095) (width 0.2) (layer "F.Cu") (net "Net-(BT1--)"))
 (segment (start 154.4355 40.428) (end 155.1356 41.1281) (width 0.2) (layer "F.Cu") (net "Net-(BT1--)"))
 (segment (start 173.5961 48.7861) (end 173.5961 37.4949) (width 0.2) (layer "F.Cu") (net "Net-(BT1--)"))
 (segment (start 180.31 68.69) (end 180.31 55.5) (width 0.2) (layer "F.Cu") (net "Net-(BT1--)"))
 (segment (start 168.0713 33.468) (end 172.0982 37.4949) (width 0.2) (layer "F.Cu") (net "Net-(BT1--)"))
 (segment (start 159.8744 36.635) (end 160.325 36.635) (width 0.2) (layer "F.Cu") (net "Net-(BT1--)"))
 (segment (start 158.7546 38.4452) (end 158.7546 37.7548) (width 0.2) (layer "F.Cu") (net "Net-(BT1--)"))
 (segment (start 173.5 79) (end 173.5 75.5) (width 0.2) (layer "F.Cu") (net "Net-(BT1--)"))
 (segment (start 154.4355 39.5845) (end 154.4355 40.428) (width 0.2) (layer "F.Cu") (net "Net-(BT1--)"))
 (segment (start 156.0717 41.1281) (end 158.7546 38.4452) (width 0.2) (layer "F.Cu") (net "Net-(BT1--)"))
 (segment (start 173.5 75.5) (end 180.31 68.69) (width 0.2) (layer "F.Cu") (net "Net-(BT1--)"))
 (segment (start 172.0982 37.4949) (end 173.5961 37.4949) (width 0.2) (layer "F.Cu") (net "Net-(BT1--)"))
 (segment (start 149.5 95) (end 160 84.5) (width 0.2) (layer "B.Cu") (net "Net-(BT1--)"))
 (segment (start 143 95) (end 138.5 99.5) (width 0.2) (layer "B.Cu") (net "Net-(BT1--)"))
 (segment (start 124.88 93.38) (end 131 99.5) (width 0.2) (layer "B.Cu") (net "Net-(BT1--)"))
 (segment (start 117.24 93.38) (end 124.88 93.38) (width 0.2) (layer "B.Cu") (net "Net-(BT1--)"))
 (segment (start 168 84.5) (end 173.5 79) (width 0.2) (layer "B.Cu") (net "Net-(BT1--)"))
 (segment (start 143 95) (end 149.5 95) (width 0.2) (layer "B.Cu") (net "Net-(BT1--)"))
 (segment (start 138.5 99.5) (end 137.5 99.5) (width 0.2) (layer "B.Cu") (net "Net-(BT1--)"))
 (segment (start 131 99.5) (end 137.5 99.5) (width 0.2) (layer "B.Cu") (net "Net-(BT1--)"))
 (segment (start 160 84.5) (end 168 84.5) (width 0.2) (layer "B.Cu") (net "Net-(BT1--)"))
 (segment (start 160.325 35.365) (end 159.9695 35.365) (width 0.2) (layer "F.Cu") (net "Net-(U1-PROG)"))
 (segment (start 159.9695 35.365) (end 155.58 39.7545) (width 0.2) (layer "F.Cu") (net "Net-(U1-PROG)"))
 (segment (start 155.58 39.7545) (end 155.58 40) (width 0.2) (layer "F.Cu") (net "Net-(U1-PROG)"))
 (segment (start 155.58 40) (end 145.42 40) (width 0.2) (layer "B.Cu") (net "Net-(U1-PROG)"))
 (segment (start 178.5 125.6) (end 176.7983 125.6) (width 0.2) (layer "F.Cu") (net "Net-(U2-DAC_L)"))
 (segment (start 176.7983 89.7983) (end 173.5 86.5) (width 0.2) (layer "F.Cu") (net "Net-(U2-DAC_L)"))
 (segment (start 176.7983 125.6) (end 176.7983 89.7983) (width 0.2) (layer "F.Cu") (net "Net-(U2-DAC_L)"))
 (segment (start 165.8405 34.095) (end 166.9583 35.2128) (width 0.2) (layer "F.Cu") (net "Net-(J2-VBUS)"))
 (segment (start 176.3 36.425) (end 176.3 35.2128) (width 0.2) (layer "F.Cu") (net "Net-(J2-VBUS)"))
 (segment (start 165.275 34.095) (end 165.8405 34.095) (width 0.2) (layer "F.Cu") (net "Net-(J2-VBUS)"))
 (segment (start 160.325 37.905) (end 160.325 38.954) (width 0.2) (layer "F.Cu") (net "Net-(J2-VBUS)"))
 (via (at 176.3 35.2128) (size 0.6) (drill 0.3) (layers "F.Cu" "B.Cu") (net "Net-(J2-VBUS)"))
 (via (at 166.9583 35.2128) (size 0.6) (drill 0.3) (layers "F.Cu" "B.Cu") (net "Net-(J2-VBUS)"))
 (via (at 160.325 38.954) (size 0.6) (drill 0.3) (layers "F.Cu" "B.Cu") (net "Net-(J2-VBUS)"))
 (segment (start 166.9583 35.2128) (end 176.3 35.2128) (width 0.2) (layer "B.Cu") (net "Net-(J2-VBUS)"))
 (segment (start 166.9583 35.2128) (end 163.2171 38.954) (width 0.2) (layer "B.Cu") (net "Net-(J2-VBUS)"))
 (segment (start 163.2171 38.954) (end 160.325 38.954) (width 0.2) (layer "B.Cu") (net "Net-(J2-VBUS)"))
 (segment (start 163.5 37.2) (end 163.5 36) (width 0.2) (layer "F.Cu") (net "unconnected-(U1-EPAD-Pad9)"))
 (segment (start 163.5 34.8) (end 163.5 36) (width 0.2) (layer "F.Cu") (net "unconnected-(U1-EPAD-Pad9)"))
 (segment (start 162.1 37.2) (end 162.1 36) (width 0.2) (layer "F.Cu") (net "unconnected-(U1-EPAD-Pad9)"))
 (segment (start 162.1 36) (end 162.1 34.8) (width 0.2) (layer "F.Cu") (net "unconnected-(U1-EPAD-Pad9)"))
 (segment (start 162.8 36) (end 162.1 36) (width 0.2) (layer "F.Cu") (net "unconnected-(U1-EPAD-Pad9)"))
 (segment (start 162.8 36) (end 162.1 36) (width 0.2) (layer "B.Cu") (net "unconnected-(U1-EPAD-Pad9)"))
 (segment (start 163.5 36) (end 162.8 36) (width 0.2) (layer "B.Cu") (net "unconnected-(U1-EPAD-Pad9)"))
 (segment (start 166 90) (end 156.5 99.5) (width 0.2) (layer "B.Cu") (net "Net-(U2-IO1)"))
 (segment (start 143 99.5) (end 149.5 99.5) (width 0.2) (layer "B.Cu") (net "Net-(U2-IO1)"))
 (segment (start 156.5 99.5) (end 149.5 99.5) (width 0.2) (layer "B.Cu") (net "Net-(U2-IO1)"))
 (segment (start 131 95) (end 137.5 95) (width 0.2) (layer "B.Cu") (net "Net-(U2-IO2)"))
 (segment (start 150 82.5) (end 137.5 95) (width 0.2) (layer "B.Cu") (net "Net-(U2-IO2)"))
 (segment (start 166 82.5) (end 150 82.5) (width 0.2) (layer "B.Cu") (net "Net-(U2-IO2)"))
 (segment (start 177.5 35.3767) (end 177.5759 35.3008) (width 0.2) (layer "F.Cu") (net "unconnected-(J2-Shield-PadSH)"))
 (segment (start 174 33.725) (end 174 33.8034) (width 0.2) (layer "F.Cu") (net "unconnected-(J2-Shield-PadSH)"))
 (segment (start 178.5 33.725) (end 177.9 33.725) (width 0.2) (layer "F.Cu") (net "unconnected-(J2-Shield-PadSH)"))
 (segment (start 177.5 36.425) (end 177.5 35.3767) (width 0.2) (layer "F.Cu") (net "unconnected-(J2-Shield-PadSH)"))
 (segment (start 176 33.725) (end 174 33.725) (width 0.2) (layer "F.Cu") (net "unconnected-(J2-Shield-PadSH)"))
 (segment (start 174 33.8034) (end 172.8267 34.9767) (width 0.2) (layer "F.Cu") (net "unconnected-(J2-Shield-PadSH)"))
 (segment (start 172.1 33.725) (end 171.5 33.725) (width 0.2) (layer "F.Cu") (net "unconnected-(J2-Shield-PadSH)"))
 (segment (start 177.5759 35.3008) (end 177.9 34.9767) (width 0.2) (layer "F.Cu") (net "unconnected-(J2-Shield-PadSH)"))
 (segment (start 177.9 33.725) (end 177.9 34.9767) (width 0.2) (layer "F.Cu") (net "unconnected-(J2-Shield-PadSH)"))
 (segment (start 177.5759 35.3008) (end 176 33.725) (width 0.2) (layer "F.Cu") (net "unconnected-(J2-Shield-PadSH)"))
 (segment (start 172.5 36.425) (end 172.5 34.9767) (width 0.2) (layer "F.Cu") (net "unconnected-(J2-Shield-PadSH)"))
 (segment (start 172.5 34.9767) (end 172.1 34.9767) (width 0.2) (layer "F.Cu") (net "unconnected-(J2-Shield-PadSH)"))
 (segment (start 172.8267 34.9767) (end 172.5 34.9767) (width 0.2) (layer "F.Cu") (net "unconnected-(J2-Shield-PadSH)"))
 (segment (start 172.1 33.725) (end 172.1 34.9767) (width 0.2) (layer "F.Cu") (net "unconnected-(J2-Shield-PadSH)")))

